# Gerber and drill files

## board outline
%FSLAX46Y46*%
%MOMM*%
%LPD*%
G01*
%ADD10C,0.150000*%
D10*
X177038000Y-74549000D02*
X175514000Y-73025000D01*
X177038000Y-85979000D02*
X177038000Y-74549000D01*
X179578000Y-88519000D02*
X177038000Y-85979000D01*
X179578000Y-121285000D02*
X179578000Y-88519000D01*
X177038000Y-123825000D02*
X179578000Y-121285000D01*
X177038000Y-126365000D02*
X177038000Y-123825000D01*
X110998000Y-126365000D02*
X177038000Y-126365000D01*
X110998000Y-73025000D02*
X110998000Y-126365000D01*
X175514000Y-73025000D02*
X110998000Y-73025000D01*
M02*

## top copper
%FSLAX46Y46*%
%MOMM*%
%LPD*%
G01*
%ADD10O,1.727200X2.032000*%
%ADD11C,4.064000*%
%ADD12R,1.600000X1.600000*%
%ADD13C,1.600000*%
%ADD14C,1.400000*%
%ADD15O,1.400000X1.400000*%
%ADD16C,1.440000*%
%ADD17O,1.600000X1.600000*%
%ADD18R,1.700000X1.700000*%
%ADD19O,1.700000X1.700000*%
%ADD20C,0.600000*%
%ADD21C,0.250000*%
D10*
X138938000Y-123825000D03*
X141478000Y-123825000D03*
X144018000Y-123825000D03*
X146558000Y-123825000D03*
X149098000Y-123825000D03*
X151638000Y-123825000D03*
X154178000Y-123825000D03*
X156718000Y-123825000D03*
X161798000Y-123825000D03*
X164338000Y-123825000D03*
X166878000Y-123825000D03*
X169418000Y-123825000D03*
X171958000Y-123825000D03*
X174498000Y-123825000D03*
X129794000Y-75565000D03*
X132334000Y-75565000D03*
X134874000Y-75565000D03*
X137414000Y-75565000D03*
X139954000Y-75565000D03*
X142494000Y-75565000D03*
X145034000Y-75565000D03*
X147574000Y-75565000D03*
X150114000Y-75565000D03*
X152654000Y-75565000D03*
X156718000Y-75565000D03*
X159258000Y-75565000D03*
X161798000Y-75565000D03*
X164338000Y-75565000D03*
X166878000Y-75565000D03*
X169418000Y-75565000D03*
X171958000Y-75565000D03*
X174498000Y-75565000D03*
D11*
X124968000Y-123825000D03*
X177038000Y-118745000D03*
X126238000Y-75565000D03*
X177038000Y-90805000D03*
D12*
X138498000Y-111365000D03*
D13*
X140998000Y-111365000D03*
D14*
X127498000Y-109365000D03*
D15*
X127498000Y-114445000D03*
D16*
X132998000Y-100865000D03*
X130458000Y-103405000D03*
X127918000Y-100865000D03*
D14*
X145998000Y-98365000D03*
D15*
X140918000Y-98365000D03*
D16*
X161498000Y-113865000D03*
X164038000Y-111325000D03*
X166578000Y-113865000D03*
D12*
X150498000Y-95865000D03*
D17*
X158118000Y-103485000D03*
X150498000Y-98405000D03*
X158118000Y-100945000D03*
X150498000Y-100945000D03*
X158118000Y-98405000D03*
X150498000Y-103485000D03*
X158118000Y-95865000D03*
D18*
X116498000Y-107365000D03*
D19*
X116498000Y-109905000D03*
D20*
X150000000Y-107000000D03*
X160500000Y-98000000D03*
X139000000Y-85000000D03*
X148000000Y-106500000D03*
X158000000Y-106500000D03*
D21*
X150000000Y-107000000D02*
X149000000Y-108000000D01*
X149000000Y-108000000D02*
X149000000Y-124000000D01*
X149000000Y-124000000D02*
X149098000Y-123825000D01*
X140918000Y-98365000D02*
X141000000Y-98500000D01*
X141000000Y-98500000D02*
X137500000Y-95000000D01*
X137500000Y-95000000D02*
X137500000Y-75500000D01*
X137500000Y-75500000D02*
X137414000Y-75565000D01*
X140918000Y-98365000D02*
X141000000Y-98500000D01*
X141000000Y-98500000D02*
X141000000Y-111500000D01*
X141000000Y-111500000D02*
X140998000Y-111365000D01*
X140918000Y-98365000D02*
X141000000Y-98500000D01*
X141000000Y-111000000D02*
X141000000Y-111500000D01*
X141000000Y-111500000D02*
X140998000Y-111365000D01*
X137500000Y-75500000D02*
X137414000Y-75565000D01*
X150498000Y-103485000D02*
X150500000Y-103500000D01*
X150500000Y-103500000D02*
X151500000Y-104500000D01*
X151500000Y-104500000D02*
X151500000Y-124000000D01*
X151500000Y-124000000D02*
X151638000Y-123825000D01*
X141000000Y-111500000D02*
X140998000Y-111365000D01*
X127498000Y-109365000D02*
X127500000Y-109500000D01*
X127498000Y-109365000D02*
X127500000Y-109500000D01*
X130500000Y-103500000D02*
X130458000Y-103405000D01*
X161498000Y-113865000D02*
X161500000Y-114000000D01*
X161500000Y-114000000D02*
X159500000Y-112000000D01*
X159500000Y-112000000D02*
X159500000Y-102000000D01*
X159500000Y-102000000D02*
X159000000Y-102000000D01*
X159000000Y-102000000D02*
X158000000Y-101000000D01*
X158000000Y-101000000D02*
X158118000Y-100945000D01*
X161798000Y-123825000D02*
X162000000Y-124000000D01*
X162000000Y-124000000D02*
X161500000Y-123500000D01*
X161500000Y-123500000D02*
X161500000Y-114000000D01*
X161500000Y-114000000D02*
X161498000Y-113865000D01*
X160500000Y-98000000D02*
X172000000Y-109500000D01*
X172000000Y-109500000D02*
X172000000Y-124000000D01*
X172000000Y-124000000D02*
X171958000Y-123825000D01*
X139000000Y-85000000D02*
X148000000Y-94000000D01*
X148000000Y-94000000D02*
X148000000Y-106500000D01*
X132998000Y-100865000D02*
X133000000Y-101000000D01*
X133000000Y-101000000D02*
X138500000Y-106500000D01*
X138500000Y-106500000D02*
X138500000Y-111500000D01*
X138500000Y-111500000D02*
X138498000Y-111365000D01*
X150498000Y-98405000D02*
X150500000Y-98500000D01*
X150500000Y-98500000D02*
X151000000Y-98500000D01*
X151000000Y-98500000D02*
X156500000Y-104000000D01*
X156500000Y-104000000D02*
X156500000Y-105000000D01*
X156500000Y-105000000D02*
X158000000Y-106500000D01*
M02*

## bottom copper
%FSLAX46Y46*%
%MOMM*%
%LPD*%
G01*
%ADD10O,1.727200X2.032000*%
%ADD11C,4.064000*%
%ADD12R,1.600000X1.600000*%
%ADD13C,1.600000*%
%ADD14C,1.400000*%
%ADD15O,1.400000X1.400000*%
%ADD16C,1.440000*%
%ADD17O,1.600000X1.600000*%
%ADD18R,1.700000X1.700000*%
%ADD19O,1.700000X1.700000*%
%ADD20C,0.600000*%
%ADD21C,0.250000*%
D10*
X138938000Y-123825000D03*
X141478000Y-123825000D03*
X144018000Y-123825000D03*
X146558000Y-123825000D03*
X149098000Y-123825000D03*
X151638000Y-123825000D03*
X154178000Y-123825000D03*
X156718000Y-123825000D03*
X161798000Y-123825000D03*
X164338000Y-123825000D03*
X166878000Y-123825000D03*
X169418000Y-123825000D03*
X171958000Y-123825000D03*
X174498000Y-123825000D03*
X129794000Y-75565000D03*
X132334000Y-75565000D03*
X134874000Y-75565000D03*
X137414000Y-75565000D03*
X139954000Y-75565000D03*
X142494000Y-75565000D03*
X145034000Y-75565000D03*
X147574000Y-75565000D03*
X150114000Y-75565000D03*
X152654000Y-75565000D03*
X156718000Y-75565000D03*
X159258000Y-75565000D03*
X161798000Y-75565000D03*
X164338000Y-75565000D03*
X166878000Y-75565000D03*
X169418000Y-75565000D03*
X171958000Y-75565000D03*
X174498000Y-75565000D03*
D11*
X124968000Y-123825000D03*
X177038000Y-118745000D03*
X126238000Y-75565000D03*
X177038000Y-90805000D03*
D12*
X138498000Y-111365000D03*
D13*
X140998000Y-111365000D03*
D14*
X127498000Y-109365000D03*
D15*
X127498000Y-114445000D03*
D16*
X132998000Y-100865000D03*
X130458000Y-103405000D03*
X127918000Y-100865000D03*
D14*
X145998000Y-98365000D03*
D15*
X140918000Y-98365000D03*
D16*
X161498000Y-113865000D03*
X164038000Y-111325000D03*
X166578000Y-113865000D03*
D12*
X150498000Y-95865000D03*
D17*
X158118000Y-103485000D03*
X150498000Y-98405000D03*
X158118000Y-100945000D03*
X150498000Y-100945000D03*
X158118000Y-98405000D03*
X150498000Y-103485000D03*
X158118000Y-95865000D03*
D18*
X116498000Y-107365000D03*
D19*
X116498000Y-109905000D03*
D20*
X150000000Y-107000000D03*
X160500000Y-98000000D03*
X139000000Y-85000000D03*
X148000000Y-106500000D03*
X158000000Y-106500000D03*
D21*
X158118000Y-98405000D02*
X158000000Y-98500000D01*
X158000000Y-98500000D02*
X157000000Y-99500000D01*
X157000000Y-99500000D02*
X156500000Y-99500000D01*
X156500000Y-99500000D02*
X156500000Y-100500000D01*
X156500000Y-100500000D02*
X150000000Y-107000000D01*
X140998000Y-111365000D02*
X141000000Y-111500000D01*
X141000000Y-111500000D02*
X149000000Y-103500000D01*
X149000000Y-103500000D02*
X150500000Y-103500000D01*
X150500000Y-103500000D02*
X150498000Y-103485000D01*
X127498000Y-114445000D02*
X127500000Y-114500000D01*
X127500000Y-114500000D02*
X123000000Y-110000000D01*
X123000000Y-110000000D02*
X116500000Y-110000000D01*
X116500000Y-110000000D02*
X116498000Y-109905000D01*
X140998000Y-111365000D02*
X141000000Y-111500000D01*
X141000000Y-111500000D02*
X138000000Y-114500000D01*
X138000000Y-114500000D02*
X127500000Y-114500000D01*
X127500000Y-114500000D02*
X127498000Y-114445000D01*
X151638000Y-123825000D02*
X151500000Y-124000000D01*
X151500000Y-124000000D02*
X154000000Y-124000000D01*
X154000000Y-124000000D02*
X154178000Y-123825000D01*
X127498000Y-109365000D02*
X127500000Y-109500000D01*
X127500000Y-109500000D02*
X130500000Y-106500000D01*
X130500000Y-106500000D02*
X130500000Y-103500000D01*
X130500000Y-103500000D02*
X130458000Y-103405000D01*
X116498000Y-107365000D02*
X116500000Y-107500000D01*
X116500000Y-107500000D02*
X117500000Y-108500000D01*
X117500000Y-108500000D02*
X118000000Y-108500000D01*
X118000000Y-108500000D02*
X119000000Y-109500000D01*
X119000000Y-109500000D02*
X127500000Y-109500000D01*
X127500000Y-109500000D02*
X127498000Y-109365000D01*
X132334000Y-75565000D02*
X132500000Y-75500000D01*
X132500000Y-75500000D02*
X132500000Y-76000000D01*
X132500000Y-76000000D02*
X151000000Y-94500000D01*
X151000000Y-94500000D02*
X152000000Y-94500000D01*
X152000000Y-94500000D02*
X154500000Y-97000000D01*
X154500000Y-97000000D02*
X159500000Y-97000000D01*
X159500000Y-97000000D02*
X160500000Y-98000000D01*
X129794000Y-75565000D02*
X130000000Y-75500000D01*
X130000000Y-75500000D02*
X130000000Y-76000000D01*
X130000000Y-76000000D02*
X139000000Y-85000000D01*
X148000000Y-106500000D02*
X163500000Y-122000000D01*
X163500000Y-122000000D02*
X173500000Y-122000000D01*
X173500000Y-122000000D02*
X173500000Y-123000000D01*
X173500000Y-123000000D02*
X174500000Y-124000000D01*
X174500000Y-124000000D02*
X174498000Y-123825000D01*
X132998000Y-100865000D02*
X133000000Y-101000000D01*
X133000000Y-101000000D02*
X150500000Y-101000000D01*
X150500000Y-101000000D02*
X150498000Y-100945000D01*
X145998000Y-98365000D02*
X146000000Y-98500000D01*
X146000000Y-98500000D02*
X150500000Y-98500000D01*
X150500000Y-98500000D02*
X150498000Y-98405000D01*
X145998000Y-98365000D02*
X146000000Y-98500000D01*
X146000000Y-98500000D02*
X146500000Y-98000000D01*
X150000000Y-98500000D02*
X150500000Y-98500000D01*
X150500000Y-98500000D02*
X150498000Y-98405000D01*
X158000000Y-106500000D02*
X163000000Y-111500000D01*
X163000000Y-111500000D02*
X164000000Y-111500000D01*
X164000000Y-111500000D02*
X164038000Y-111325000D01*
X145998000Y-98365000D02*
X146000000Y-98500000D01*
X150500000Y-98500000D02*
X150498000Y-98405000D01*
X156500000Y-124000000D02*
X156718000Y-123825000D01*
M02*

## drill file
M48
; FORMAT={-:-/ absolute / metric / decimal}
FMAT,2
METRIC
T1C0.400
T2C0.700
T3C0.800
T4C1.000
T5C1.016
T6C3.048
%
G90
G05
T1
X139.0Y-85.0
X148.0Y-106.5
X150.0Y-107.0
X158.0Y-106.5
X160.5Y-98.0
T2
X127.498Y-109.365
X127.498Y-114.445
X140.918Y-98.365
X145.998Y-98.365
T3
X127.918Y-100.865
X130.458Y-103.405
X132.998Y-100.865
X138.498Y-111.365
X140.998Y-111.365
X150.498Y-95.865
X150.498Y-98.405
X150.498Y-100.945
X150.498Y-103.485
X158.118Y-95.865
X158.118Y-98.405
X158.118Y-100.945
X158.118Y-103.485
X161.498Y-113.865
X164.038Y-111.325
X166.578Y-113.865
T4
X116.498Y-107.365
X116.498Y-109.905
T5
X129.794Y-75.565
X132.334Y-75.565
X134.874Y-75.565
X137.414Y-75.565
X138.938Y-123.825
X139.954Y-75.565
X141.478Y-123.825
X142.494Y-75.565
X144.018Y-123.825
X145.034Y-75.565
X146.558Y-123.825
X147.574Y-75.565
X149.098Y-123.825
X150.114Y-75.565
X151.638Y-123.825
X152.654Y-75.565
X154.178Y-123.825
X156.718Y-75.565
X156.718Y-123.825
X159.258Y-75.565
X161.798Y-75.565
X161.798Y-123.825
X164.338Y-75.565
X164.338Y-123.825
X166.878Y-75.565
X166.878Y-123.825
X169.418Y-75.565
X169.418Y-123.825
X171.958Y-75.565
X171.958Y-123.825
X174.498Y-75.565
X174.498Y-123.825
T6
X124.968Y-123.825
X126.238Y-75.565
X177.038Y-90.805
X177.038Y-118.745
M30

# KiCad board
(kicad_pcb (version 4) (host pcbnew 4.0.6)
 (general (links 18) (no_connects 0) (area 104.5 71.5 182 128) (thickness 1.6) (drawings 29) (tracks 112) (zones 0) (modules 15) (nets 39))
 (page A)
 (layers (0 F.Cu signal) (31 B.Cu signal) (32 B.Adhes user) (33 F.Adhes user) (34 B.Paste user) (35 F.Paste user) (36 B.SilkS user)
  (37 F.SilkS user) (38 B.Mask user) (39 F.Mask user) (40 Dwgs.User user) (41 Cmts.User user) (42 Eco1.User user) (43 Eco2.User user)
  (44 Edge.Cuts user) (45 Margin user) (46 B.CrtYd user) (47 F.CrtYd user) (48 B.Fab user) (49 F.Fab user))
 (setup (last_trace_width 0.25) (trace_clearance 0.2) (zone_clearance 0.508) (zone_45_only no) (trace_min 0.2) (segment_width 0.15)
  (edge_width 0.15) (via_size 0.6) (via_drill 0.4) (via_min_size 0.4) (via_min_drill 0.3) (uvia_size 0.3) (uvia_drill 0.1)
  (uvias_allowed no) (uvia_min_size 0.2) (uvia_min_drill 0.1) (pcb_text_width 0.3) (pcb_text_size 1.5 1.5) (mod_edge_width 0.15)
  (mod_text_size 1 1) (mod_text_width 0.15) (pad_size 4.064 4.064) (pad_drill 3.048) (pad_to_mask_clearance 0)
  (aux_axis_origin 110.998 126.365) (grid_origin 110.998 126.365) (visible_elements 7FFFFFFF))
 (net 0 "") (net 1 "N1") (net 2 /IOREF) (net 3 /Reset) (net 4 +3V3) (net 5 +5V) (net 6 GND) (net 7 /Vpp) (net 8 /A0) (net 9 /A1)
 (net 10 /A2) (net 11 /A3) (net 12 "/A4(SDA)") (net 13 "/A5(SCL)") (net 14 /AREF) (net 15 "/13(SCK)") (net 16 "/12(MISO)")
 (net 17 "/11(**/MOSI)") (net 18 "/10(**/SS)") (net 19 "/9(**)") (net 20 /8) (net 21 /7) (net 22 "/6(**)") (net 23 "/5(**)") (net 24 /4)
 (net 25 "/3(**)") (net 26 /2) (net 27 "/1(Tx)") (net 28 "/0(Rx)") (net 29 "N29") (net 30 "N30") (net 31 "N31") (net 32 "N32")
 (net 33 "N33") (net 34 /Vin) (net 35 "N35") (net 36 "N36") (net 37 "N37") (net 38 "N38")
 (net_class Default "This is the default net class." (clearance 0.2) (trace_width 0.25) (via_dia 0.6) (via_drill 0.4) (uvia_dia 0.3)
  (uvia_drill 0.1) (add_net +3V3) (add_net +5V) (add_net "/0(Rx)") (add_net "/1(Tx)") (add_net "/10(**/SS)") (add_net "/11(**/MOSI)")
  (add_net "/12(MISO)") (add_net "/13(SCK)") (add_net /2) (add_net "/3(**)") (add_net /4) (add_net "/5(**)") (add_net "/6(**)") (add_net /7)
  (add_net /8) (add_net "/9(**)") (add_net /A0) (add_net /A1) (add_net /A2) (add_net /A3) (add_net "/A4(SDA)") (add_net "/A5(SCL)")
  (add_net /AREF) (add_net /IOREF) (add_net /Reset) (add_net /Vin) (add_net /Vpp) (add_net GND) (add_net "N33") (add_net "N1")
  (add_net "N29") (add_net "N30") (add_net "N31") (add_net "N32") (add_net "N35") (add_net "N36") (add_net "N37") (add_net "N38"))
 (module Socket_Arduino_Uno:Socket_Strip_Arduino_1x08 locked (layer F.Cu) (at 138.938 123.825)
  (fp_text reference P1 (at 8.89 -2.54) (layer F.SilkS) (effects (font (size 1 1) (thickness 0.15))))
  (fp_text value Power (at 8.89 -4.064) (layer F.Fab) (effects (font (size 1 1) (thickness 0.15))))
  (pad 1 thru_hole oval (at 0 0) (size 1.7272 2.032) (drill 1.016) (layers *.Cu *.Mask F.SilkS) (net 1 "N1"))
  (pad 2 thru_hole oval (at 2.54 0) (size 1.7272 2.032) (drill 1.016) (layers *.Cu *.Mask F.SilkS) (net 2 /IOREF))
  (pad 3 thru_hole oval (at 5.08 0) (size 1.7272 2.032) (drill 1.016) (layers *.Cu *.Mask F.SilkS) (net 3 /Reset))
  (pad 4 thru_hole oval (at 7.62 0) (size 1.7272 2.032) (drill 1.016) (layers *.Cu *.Mask F.SilkS) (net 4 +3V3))
  (pad 5 thru_hole oval (at 10.16 0) (size 1.7272 2.032) (drill 1.016) (layers *.Cu *.Mask F.SilkS) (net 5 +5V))
  (pad 6 thru_hole oval (at 12.7 0) (size 1.7272 2.032) (drill 1.016) (layers *.Cu *.Mask F.SilkS) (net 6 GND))
  (pad 7 thru_hole oval (at 15.24 0) (size 1.7272 2.032) (drill 1.016) (layers *.Cu *.Mask F.SilkS) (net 6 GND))
  (pad 8 thru_hole oval (at 17.78 0) (size 1.7272 2.032) (drill 1.016) (layers *.Cu *.Mask F.SilkS) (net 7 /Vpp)))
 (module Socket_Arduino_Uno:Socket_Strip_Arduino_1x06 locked (layer F.Cu) (at 161.798 123.825)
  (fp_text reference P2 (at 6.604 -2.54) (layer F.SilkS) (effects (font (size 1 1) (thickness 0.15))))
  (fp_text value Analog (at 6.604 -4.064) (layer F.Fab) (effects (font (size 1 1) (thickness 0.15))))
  (pad 1 thru_hole oval (at 0 0) (size 1.7272 2.032) (drill 1.016) (layers *.Cu *.Mask F.SilkS) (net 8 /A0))
  (pad 2 thru_hole oval (at 2.54 0) (size 1.7272 2.032) (drill 1.016) (layers *.Cu *.Mask F.SilkS) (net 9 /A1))
  (pad 3 thru_hole oval (at 5.08 0) (size 1.7272 2.032) (drill 1.016) (layers *.Cu *.Mask F.SilkS) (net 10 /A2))
  (pad 4 thru_hole oval (at 7.62 0) (size 1.7272 2.032) (drill 1.016) (layers *.Cu *.Mask F.SilkS) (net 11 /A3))
  (pad 5 thru_hole oval (at 10.16 0) (size 1.7272 2.032) (drill 1.016) (layers *.Cu *.Mask F.SilkS) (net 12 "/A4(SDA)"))
  (pad 6 thru_hole oval (at 12.7 0) (size 1.7272 2.032) (drill 1.016) (layers *.Cu *.Mask F.SilkS) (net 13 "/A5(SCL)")))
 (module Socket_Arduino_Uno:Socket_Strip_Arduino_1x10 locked (layer F.Cu) (at 129.794 75.565)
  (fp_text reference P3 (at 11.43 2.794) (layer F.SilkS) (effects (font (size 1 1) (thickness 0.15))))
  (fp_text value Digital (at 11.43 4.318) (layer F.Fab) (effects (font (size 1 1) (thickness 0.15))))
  (pad 1 thru_hole oval (at 0 0) (size 1.7272 2.032) (drill 1.016) (layers *.Cu *.Mask F.SilkS) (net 13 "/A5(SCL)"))
  (pad 2 thru_hole oval (at 2.54 0) (size 1.7272 2.032) (drill 1.016) (layers *.Cu *.Mask F.SilkS) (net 12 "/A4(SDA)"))
  (pad 3 thru_hole oval (at 5.08 0) (size 1.7272 2.032) (drill 1.016) (layers *.Cu *.Mask F.SilkS) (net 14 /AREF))
  (pad 4 thru_hole oval (at 7.62 0) (size 1.7272 2.032) (drill 1.016) (layers *.Cu *.Mask F.SilkS) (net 6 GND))
  (pad 5 thru_hole oval (at 10.16 0) (size 1.7272 2.032) (drill 1.016) (layers *.Cu *.Mask F.SilkS) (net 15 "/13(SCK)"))
  (pad 6 thru_hole oval (at 12.7 0) (size 1.7272 2.032) (drill 1.016) (layers *.Cu *.Mask F.SilkS) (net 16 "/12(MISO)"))
  (pad 7 thru_hole oval (at 15.24 0) (size 1.7272 2.032) (drill 1.016) (layers *.Cu *.Mask F.SilkS) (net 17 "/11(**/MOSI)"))
  (pad 8 thru_hole oval (at 17.78 0) (size 1.7272 2.032) (drill 1.016) (layers *.Cu *.Mask F.SilkS) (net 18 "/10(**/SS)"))
  (pad 9 thru_hole oval (at 20.32 0) (size 1.7272 2.032) (drill 1.016) (layers *.Cu *.Mask F.SilkS) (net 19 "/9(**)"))
  (pad 10 thru_hole oval (at 22.86 0) (size 1.7272 2.032) (drill 1.016) (layers *.Cu *.Mask F.SilkS) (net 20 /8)))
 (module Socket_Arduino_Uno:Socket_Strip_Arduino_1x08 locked (layer F.Cu) (at 156.718 75.565)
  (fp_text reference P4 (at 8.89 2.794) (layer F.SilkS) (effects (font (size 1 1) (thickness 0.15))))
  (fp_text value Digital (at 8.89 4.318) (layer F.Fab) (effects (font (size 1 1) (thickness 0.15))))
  (pad 1 thru_hole oval (at 0 0) (size 1.7272 2.032) (drill 1.016) (layers *.Cu *.Mask F.SilkS) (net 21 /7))
  (pad 2 thru_hole oval (at 2.54 0) (size 1.7272 2.032) (drill 1.016) (layers *.Cu *.Mask F.SilkS) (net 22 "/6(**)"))
  (pad 3 thru_hole oval (at 5.08 0) (size 1.7272 2.032) (drill 1.016) (layers *.Cu *.Mask F.SilkS) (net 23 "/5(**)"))
  (pad 4 thru_hole oval (at 7.62 0) (size 1.7272 2.032) (drill 1.016) (layers *.Cu *.Mask F.SilkS) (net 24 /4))
  (pad 5 thru_hole oval (at 10.16 0) (size 1.7272 2.032) (drill 1.016) (layers *.Cu *.Mask F.SilkS) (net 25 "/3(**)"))
  (pad 6 thru_hole oval (at 12.7 0) (size 1.7272 2.032) (drill 1.016) (layers *.Cu *.Mask F.SilkS) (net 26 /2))
  (pad 7 thru_hole oval (at 15.24 0) (size 1.7272 2.032) (drill 1.016) (layers *.Cu *.Mask F.SilkS) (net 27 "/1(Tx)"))
  (pad 8 thru_hole oval (at 17.78 0) (size 1.7272 2.032) (drill 1.016) (layers *.Cu *.Mask F.SilkS) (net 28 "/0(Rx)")))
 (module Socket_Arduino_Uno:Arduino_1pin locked (layer F.Cu) (at 124.968 123.825)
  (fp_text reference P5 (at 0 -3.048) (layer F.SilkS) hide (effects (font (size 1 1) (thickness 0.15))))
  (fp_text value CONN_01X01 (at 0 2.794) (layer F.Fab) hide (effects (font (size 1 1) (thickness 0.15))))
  (pad 1 thru_hole circle (at 0 0) (size 4.064 4.064) (drill 3.048) (layers *.Cu *.Mask F.SilkS) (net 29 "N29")))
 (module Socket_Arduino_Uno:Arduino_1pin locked (layer F.Cu) (at 177.038 118.745)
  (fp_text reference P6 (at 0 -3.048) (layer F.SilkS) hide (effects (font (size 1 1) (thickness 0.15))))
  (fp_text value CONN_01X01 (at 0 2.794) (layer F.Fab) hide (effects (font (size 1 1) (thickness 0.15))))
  (pad 1 thru_hole circle (at 0 0) (size 4.064 4.064) (drill 3.048) (layers *.Cu *.Mask F.SilkS) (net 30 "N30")))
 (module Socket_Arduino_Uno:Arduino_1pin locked (layer F.Cu) (at 126.238 75.565)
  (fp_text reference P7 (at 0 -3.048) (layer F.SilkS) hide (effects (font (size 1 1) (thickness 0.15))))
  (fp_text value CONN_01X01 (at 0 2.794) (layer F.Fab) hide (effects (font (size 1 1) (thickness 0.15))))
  (pad 1 thru_hole circle (at 0 0) (size 4.064 4.064) (drill 3.048) (layers *.Cu *.Mask F.SilkS) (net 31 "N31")))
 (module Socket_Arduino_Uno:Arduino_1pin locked (layer F.Cu) (at 177.038 90.805)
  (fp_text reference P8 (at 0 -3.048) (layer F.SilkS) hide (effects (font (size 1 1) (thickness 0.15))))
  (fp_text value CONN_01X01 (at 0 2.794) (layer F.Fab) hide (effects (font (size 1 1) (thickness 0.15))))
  (pad 1 thru_hole circle (at 0 0) (size 4.064 4.064) (drill 3.048) (layers *.Cu *.Mask F.SilkS) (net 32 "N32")))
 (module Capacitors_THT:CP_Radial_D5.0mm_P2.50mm (layer F.Cu) (at 138.498 111.365)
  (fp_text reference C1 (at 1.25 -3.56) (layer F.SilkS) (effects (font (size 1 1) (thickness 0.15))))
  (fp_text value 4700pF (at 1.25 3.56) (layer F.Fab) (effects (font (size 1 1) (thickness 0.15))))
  (pad 1 thru_hole rect (at 0 0) (size 1.6 1.6) (drill 0.8) (layers *.Cu *.Mask) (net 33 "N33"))
  (pad 2 thru_hole circle (at 2.5 0) (size 1.6 1.6) (drill 0.8) (layers *.Cu *.Mask) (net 6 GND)))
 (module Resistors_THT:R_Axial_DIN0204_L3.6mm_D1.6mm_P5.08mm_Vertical (layer F.Cu) (at 127.498 109.365 270)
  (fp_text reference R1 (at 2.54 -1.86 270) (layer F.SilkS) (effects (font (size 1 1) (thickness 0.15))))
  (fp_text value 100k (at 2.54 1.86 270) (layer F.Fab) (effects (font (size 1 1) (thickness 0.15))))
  (pad 1 thru_hole circle (at 0 0 270) (size 1.4 1.4) (drill 0.7) (layers *.Cu *.Mask) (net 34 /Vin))
  (pad 2 thru_hole oval (at 5.08 0 270) (size 1.4 1.4) (drill 0.7) (layers *.Cu *.Mask) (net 6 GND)))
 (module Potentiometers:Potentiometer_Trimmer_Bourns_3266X (layer F.Cu) (at 132.998 100.865)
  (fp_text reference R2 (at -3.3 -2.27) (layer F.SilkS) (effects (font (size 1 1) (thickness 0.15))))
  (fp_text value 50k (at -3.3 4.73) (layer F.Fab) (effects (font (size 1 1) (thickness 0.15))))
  (pad 1 thru_hole circle (at 0 0) (size 1.44 1.44) (drill 0.8) (layers *.Cu *.Mask) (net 33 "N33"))
  (pad 2 thru_hole circle (at -2.54 2.54) (size 1.44 1.44) (drill 0.8) (layers *.Cu *.Mask) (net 34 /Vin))
  (pad 3 thru_hole circle (at -5.08 0) (size 1.44 1.44) (drill 0.8) (layers *.Cu *.Mask)))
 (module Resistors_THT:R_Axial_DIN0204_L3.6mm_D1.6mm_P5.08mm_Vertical (layer F.Cu) (at 145.998 98.365 180)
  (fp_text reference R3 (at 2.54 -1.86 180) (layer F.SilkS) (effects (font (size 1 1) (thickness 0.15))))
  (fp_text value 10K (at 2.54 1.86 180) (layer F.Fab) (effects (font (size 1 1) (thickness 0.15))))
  (pad 1 thru_hole circle (at 0 0 180) (size 1.4 1.4) (drill 0.7) (layers *.Cu *.Mask) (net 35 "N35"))
  (pad 2 thru_hole oval (at 5.08 0 180) (size 1.4 1.4) (drill 0.7) (layers *.Cu *.Mask) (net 6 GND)))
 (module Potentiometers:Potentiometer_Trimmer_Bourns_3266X (layer F.Cu) (at 161.498 113.865 180)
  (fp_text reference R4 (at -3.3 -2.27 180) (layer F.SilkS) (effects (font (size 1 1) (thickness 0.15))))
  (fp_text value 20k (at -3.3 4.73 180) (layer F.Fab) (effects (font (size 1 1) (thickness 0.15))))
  (pad 1 thru_hole circle (at 0 0 180) (size 1.44 1.44) (drill 0.8) (layers *.Cu *.Mask) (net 8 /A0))
  (pad 2 thru_hole circle (at -2.54 2.54 180) (size 1.44 1.44) (drill 0.8) (layers *.Cu *.Mask) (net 35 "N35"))
  (pad 3 thru_hole circle (at -5.08 0 180) (size 1.44 1.44) (drill 0.8) (layers *.Cu *.Mask)))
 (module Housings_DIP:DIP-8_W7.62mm (layer F.Cu) (at 150.498 95.865)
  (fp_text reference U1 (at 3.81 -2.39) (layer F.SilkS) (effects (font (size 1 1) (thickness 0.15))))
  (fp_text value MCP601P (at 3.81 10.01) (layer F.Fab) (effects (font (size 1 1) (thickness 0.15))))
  (pad 1 thru_hole rect (at 0 0) (size 1.6 1.6) (drill 0.8) (layers *.Cu *.Mask) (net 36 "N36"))
  (pad 5 thru_hole oval (at 7.62 7.62) (size 1.6 1.6) (drill 0.8) (layers *.Cu *.Mask) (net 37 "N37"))
  (pad 2 thru_hole oval (at 0 2.54) (size 1.6 1.6) (drill 0.8) (layers *.Cu *.Mask) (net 35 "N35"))
  (pad 6 thru_hole oval (at 7.62 5.08) (size 1.6 1.6) (drill 0.8) (layers *.Cu *.Mask) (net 8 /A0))
  (pad 3 thru_hole oval (at 0 5.08) (size 1.6 1.6) (drill 0.8) (layers *.Cu *.Mask) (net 33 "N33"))
  (pad 7 thru_hole oval (at 7.62 2.54) (size 1.6 1.6) (drill 0.8) (layers *.Cu *.Mask) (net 5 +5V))
  (pad 4 thru_hole oval (at 0 7.62) (size 1.6 1.6) (drill 0.8) (layers *.Cu *.Mask) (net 6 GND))
  (pad 8 thru_hole oval (at 7.62 0) (size 1.6 1.6) (drill 0.8) (layers *.Cu *.Mask) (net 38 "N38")))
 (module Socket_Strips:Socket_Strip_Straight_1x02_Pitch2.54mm (layer F.Cu) (at 116.498 107.365)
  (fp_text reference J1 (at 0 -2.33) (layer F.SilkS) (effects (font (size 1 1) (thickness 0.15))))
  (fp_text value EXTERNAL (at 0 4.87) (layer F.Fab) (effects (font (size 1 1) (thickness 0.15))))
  (pad 1 thru_hole rect (at 0 0) (size 1.7 1.7) (drill 1) (layers *.Cu *.Mask) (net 34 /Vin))
  (pad 2 thru_hole oval (at 0 2.54) (size 1.7 1.7) (drill 1) (layers *.Cu *.Mask) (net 6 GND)))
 (gr_line (start 177.038 74.549) (end 175.514 73.025) (angle 90) (layer Edge.Cuts) (width 0.15))
 (gr_line (start 177.038 85.979) (end 177.038 74.549) (angle 90) (layer Edge.Cuts) (width 0.15))
 (gr_line (start 179.578 88.519) (end 177.038 85.979) (angle 90) (layer Edge.Cuts) (width 0.15))
 (gr_line (start 179.578 121.285) (end 179.578 88.519) (angle 90) (layer Edge.Cuts) (width 0.15))
 (gr_line (start 177.038 123.825) (end 179.578 121.285) (angle 90) (layer Edge.Cuts) (width 0.15))
 (gr_line (start 177.038 126.365) (end 177.038 123.825) (angle 90) (layer Edge.Cuts) (width 0.15))
 (gr_line (start 110.998 126.365) (end 177.038 126.365) (angle 90) (layer Edge.Cuts) (width 0.15))
 (gr_line (start 110.998 73.025) (end 110.998 126.365) (angle 90) (layer Edge.Cuts) (width 0.15))
 (gr_line (start 175.514 73.025) (end 110.998 73.025) (angle 90) (layer Edge.Cuts) (width 0.15))
 (segment (start 158.118 98.405) (end 158 98.5) (width 0.25) (layer B.Cu) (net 5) (status 80000))
 (segment (start 158 98.5) (end 157 99.5) (width 0.25) (layer B.Cu) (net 5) (status 80000))
 (segment (start 157 99.5) (end 156.5 99.5) (width 0.25) (layer B.Cu) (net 5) (status 80000))
 (segment (start 156.5 99.5) (end 156.5 100.5) (width 0.25) (layer B.Cu) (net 5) (status 80000))
 (segment (start 156.5 100.5) (end 150 107) (width 0.25) (layer B.Cu) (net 5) (status 80000))
 (via (at 150 107) (size 0.6) (layers F.Cu B.Cu) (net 5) (status 80000))
 (segment (start 150 107) (end 149 108) (width 0.25) (layer F.Cu) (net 5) (status 80000))
 (segment (start 149 108) (end 149 124) (width 0.25) (layer F.Cu) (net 5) (status 80000))
 (segment (start 149 124) (end 149.098 123.825) (width 0.25) (layer F.Cu) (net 5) (status 80000))
 (segment (start 140.918 98.365) (end 141 98.5) (width 0.25) (layer F.Cu) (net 6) (status 80000))
 (segment (start 141 98.5) (end 137.5 95) (width 0.25) (layer F.Cu) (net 6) (status 80000))
 (segment (start 137.5 95) (end 137.5 75.5) (width 0.25) (layer F.Cu) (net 6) (status 80000))
 (segment (start 137.5 75.5) (end 137.414 75.565) (width 0.25) (layer F.Cu) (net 6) (status 80000))
 (segment (start 140.918 98.365) (end 141 98.5) (width 0.25) (layer F.Cu) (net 6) (status 80000))
 (segment (start 141 98.5) (end 141 111.5) (width 0.25) (layer F.Cu) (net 6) (status 80000))
 (segment (start 141 111.5) (end 140.998 111.365) (width 0.25) (layer F.Cu) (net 6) (status 80000))
 (segment (start 140.918 98.365) (end 141 98.5) (width 0.25) (layer F.Cu) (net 6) (status 80000))
 (segment (start 141 111) (end 141 111.5) (width 0.25) (layer F.Cu) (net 6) (status 80000))
 (segment (start 141 111.5) (end 140.998 111.365) (width 0.25) (layer F.Cu) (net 6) (status 80000))
 (segment (start 140.998 111.365) (end 141 111.5) (width 0.25) (layer B.Cu) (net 6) (status 80000))
 (segment (start 141 111.5) (end 149 103.5) (width 0.25) (layer B.Cu) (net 6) (status 80000))
 (segment (start 149 103.5) (end 150.5 103.5) (width 0.25) (layer B.Cu) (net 6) (status 80000))
 (segment (start 150.5 103.5) (end 150.498 103.485) (width 0.25) (layer B.Cu) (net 6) (status 80000))
 (segment (start 137.5 75.5) (end 137.414 75.565) (width 0.25) (layer F.Cu) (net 6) (status 80000))
 (segment (start 127.498 114.445) (end 127.5 114.5) (width 0.25) (layer B.Cu) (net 6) (status 80000))
 (segment (start 127.5 114.5) (end 123 110) (width 0.25) (layer B.Cu) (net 6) (status 80000))
 (segment (start 123 110) (end 116.5 110) (width 0.25) (layer B.Cu) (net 6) (status 80000))
 (segment (start 116.5 110) (end 116.498 109.905) (width 0.25) (layer B.Cu) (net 6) (status 80000))
 (segment (start 140.998 111.365) (end 141 111.5) (width 0.25) (layer B.Cu) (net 6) (status 80000))
 (segment (start 141 111.5) (end 138 114.5) (width 0.25) (layer B.Cu) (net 6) (status 80000))
 (segment (start 138 114.5) (end 127.5 114.5) (width 0.25) (layer B.Cu) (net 6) (status 80000))
 (segment (start 127.5 114.5) (end 127.498 114.445) (width 0.25) (layer B.Cu) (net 6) (status 80000))
 (segment (start 150.498 103.485) (end 150.5 103.5) (width 0.25) (layer F.Cu) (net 6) (status 80000))
 (segment (start 150.5 103.5) (end 151.5 104.5) (width 0.25) (layer F.Cu) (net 6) (status 80000))
 (segment (start 151.5 104.5) (end 151.5 124) (width 0.25) (layer F.Cu) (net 6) (status 80000))
 (segment (start 151.5 124) (end 151.638 123.825) (width 0.25) (layer F.Cu) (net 6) (status 80000))
 (segment (start 141 111.5) (end 140.998 111.365) (width 0.25) (layer F.Cu) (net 6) (status 80000))
 (segment (start 151.638 123.825) (end 151.5 124) (width 0.25) (layer B.Cu) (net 6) (status 80000))
 (segment (start 151.5 124) (end 154 124) (width 0.25) (layer B.Cu) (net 6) (status 80000))
 (segment (start 154 124) (end 154.178 123.825) (width 0.25) (layer B.Cu) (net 6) (status 80000))
 (segment (start 127.498 109.365) (end 127.5 109.5) (width 0.25) (layer B.Cu) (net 34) (status 80000))
 (segment (start 127.5 109.5) (end 130.5 106.5) (width 0.25) (layer B.Cu) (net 34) (status 80000))
 (segment (start 130.5 106.5) (end 130.5 103.5) (width 0.25) (layer B.Cu) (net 34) (status 80000))
 (segment (start 130.5 103.5) (end 130.458 103.405) (width 0.25) (layer B.Cu) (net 34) (status 80000))
 (segment (start 127.498 109.365) (end 127.5 109.5) (width 0.25) (layer F.Cu) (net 34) (status 80000))
 (segment (start 127.498 109.365) (end 127.5 109.5) (width 0.25) (layer F.Cu) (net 34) (status 80000))
 (segment (start 130.5 103.5) (end 130.458 103.405) (width 0.25) (layer F.Cu) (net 34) (status 80000))
 (segment (start 116.498 107.365) (end 116.5 107.5) (width 0.25) (layer B.Cu) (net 34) (status 80000))
 (segment (start 116.5 107.5) (end 117.5 108.5) (width 0.25) (layer B.Cu) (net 34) (status 80000))
 (segment (start 117.5 108.5) (end 118 108.5) (width 0.25) (layer B.Cu) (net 34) (status 80000))
 (segment (start 118 108.5) (end 119 109.5) (width 0.25) (layer B.Cu) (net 34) (status 80000))
 (segment (start 119 109.5) (end 127.5 109.5) (width 0.25) (layer B.Cu) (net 34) (status 80000))
 (segment (start 127.5 109.5) (end 127.498 109.365) (width 0.25) (layer B.Cu) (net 34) (status 80000))
 (segment (start 161.498 113.865) (end 161.5 114) (width 0.25) (layer F.Cu) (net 8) (status 80000))
 (segment (start 161.5 114) (end 159.5 112) (width 0.25) (layer F.Cu) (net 8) (status 80000))
 (segment (start 159.5 112) (end 159.5 102) (width 0.25) (layer F.Cu) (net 8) (status 80000))
 (segment (start 159.5 102) (end 159 102) (width 0.25) (layer F.Cu) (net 8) (status 80000))
 (segment (start 159 102) (end 158 101) (width 0.25) (layer F.Cu) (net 8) (status 80000))
 (segment (start 158 101) (end 158.118 100.945) (width 0.25) (layer F.Cu) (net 8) (status 80000))
 (segment (start 161.798 123.825) (end 162 124) (width 0.25) (layer F.Cu) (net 8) (status 80000))
 (segment (start 162 124) (end 161.5 123.5) (width 0.25) (layer F.Cu) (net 8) (status 80000))
 (segment (start 161.5 123.5) (end 161.5 114) (width 0.25) (layer F.Cu) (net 8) (status 80000))
 (segment (start 161.5 114) (end 161.498 113.865) (width 0.25) (layer F.Cu) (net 8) (status 80000))
 (segment (start 132.334 75.565) (end 132.5 75.5) (width 0.25) (layer B.Cu) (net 12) (status 80000))
 (segment (start 132.5 75.5) (end 132.5 76) (width 0.25) (layer B.Cu) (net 12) (status 80000))
 (segment (start 132.5 76) (end 151 94.5) (width 0.25) (layer B.Cu) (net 12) (status 80000))
 (segment (start 151 94.5) (end 152 94.5) (width 0.25) (layer B.Cu) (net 12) (status 80000))
 (segment (start 152 94.5) (end 154.5 97) (width 0.25) (layer B.Cu) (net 12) (status 80000))
 (segment (start 154.5 97) (end 159.5 97) (width 0.25) (layer B.Cu) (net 12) (status 80000))
 (segment (start 159.5 97) (end 160.5 98) (width 0.25) (layer B.Cu) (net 12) (status 80000))
 (via (at 160.5 98) (size 0.6) (layers F.Cu B.Cu) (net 12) (status 80000))
 (segment (start 160.5 98) (end 172 109.5) (width 0.25) (layer F.Cu) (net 12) (status 80000))
 (segment (start 172 109.5) (end 172 124) (width 0.25) (layer F.Cu) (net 12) (status 80000))
 (segment (start 172 124) (end 171.958 123.825) (width 0.25) (layer F.Cu) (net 12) (status 80000))
 (segment (start 129.794 75.565) (end 130 75.5) (width 0.25) (layer B.Cu) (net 13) (status 80000))
 (segment (start 130 75.5) (end 130 76) (width 0.25) (layer B.Cu) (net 13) (status 80000))
 (segment (start 130 76) (end 139 85) (width 0.25) (layer B.Cu) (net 13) (status 80000))
 (via (at 139 85) (size 0.6) (layers F.Cu B.Cu) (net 13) (status 80000))
 (segment (start 139 85) (end 148 94) (width 0.25) (layer F.Cu) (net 13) (status 80000))
 (segment (start 148 94) (end 148 106.5) (width 0.25) (layer F.Cu) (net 13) (status 80000))
 (via (at 148 106.5) (size 0.6) (layers F.Cu B.Cu) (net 13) (status 80000))
 (segment (start 148 106.5) (end 163.5 122) (width 0.25) (layer B.Cu) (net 13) (status 80000))
 (segment (start 163.5 122) (end 173.5 122) (width 0.25) (layer B.Cu) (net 13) (status 80000))
 (segment (start 173.5 122) (end 173.5 123) (width 0.25) (layer B.Cu) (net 13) (status 80000))
 (segment (start 173.5 123) (end 174.5 124) (width 0.25) (layer B.Cu) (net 13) (status 80000))
 (segment (start 174.5 124) (end 174.498 123.825) (width 0.25) (layer B.Cu) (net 13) (status 80000))
 (segment (start 132.998 100.865) (end 133 101) (width 0.25) (layer F.Cu) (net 33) (status 80000))
 (segment (start 133 101) (end 138.5 106.5) (width 0.25) (layer F.Cu) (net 33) (status 80000))
 (segment (start 138.5 106.5) (end 138.5 111.5) (width 0.25) (layer F.Cu) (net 33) (status 80000))
 (segment (start 138.5 111.5) (end 138.498 111.365) (width 0.25) (layer F.Cu) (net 33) (status 80000))
 (segment (start 132.998 100.865) (end 133 101) (width 0.25) (layer B.Cu) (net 33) (status 80000))
 (segment (start 133 101) (end 150.5 101) (width 0.25) (layer B.Cu) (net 33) (status 80000))
 (segment (start 150.5 101) (end 150.498 100.945) (width 0.25) (layer B.Cu) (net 33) (status 80000))
 (segment (start 145.998 98.365) (end 146 98.5) (width 0.25) (layer B.Cu) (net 35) (status 80000))
 (segment (start 146 98.5) (end 150.5 98.5) (width 0.25) (layer B.Cu) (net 35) (status 80000))
 (segment (start 150.5 98.5) (end 150.498 98.405) (width 0.25) (layer B.Cu) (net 35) (status 80000))
 (segment (start 145.998 98.365) (end 146 98.5) (width 0.25) (layer B.Cu) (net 35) (status 80000))
 (segment (start 146 98.5) (end 146.5 98) (width 0.25) (layer B.Cu) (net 35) (status 80000))
 (segment (start 150 98.5) (end 150.5 98.5) (width 0.25) (layer B.Cu) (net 35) (status 80000))
 (segment (start 150.5 98.5) (end 150.498 98.405) (width 0.25) (layer B.Cu) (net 35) (status 80000))
 (segment (start 150.498 98.405) (end 150.5 98.5) (width 0.25) (layer F.Cu) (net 35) (status 80000))
 (segment (start 150.5 98.5) (end 151 98.5) (width 0.25) (layer F.Cu) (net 35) (status 80000))
 (segment (start 151 98.5) (end 156.5 104) (width 0.25) (layer F.Cu) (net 35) (status 80000))
 (segment (start 156.5 104) (end 156.5 105) (width 0.25) (layer F.Cu) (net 35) (status 80000))
 (segment (start 156.5 105) (end 158 106.5) (width 0.25) (layer F.Cu) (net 35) (status 80000))
 (via (at 158 106.5) (size 0.6) (layers F.Cu B.Cu) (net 35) (status 80000))
 (segment (start 158 106.5) (end 163 111.5) (width 0.25) (layer B.Cu) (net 35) (status 80000))
 (segment (start 163 111.5) (end 164 111.5) (width 0.25) (layer B.Cu) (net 35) (status 80000))
 (segment (start 164 111.5) (end 164.038 111.325) (width 0.25) (layer B.Cu) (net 35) (status 80000))
 (segment (start 145.998 98.365) (end 146 98.5) (width 0.25) (layer B.Cu) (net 35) (status 80030))
 (segment (start 150.5 98.5) (end 150.498 98.405) (width 0.25) (layer B.Cu) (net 35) (status 80000))
 (segment (start 156.5 124) (end 156.718 123.825) (width 0.25) (layer B.Cu) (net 7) (status 80000)))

